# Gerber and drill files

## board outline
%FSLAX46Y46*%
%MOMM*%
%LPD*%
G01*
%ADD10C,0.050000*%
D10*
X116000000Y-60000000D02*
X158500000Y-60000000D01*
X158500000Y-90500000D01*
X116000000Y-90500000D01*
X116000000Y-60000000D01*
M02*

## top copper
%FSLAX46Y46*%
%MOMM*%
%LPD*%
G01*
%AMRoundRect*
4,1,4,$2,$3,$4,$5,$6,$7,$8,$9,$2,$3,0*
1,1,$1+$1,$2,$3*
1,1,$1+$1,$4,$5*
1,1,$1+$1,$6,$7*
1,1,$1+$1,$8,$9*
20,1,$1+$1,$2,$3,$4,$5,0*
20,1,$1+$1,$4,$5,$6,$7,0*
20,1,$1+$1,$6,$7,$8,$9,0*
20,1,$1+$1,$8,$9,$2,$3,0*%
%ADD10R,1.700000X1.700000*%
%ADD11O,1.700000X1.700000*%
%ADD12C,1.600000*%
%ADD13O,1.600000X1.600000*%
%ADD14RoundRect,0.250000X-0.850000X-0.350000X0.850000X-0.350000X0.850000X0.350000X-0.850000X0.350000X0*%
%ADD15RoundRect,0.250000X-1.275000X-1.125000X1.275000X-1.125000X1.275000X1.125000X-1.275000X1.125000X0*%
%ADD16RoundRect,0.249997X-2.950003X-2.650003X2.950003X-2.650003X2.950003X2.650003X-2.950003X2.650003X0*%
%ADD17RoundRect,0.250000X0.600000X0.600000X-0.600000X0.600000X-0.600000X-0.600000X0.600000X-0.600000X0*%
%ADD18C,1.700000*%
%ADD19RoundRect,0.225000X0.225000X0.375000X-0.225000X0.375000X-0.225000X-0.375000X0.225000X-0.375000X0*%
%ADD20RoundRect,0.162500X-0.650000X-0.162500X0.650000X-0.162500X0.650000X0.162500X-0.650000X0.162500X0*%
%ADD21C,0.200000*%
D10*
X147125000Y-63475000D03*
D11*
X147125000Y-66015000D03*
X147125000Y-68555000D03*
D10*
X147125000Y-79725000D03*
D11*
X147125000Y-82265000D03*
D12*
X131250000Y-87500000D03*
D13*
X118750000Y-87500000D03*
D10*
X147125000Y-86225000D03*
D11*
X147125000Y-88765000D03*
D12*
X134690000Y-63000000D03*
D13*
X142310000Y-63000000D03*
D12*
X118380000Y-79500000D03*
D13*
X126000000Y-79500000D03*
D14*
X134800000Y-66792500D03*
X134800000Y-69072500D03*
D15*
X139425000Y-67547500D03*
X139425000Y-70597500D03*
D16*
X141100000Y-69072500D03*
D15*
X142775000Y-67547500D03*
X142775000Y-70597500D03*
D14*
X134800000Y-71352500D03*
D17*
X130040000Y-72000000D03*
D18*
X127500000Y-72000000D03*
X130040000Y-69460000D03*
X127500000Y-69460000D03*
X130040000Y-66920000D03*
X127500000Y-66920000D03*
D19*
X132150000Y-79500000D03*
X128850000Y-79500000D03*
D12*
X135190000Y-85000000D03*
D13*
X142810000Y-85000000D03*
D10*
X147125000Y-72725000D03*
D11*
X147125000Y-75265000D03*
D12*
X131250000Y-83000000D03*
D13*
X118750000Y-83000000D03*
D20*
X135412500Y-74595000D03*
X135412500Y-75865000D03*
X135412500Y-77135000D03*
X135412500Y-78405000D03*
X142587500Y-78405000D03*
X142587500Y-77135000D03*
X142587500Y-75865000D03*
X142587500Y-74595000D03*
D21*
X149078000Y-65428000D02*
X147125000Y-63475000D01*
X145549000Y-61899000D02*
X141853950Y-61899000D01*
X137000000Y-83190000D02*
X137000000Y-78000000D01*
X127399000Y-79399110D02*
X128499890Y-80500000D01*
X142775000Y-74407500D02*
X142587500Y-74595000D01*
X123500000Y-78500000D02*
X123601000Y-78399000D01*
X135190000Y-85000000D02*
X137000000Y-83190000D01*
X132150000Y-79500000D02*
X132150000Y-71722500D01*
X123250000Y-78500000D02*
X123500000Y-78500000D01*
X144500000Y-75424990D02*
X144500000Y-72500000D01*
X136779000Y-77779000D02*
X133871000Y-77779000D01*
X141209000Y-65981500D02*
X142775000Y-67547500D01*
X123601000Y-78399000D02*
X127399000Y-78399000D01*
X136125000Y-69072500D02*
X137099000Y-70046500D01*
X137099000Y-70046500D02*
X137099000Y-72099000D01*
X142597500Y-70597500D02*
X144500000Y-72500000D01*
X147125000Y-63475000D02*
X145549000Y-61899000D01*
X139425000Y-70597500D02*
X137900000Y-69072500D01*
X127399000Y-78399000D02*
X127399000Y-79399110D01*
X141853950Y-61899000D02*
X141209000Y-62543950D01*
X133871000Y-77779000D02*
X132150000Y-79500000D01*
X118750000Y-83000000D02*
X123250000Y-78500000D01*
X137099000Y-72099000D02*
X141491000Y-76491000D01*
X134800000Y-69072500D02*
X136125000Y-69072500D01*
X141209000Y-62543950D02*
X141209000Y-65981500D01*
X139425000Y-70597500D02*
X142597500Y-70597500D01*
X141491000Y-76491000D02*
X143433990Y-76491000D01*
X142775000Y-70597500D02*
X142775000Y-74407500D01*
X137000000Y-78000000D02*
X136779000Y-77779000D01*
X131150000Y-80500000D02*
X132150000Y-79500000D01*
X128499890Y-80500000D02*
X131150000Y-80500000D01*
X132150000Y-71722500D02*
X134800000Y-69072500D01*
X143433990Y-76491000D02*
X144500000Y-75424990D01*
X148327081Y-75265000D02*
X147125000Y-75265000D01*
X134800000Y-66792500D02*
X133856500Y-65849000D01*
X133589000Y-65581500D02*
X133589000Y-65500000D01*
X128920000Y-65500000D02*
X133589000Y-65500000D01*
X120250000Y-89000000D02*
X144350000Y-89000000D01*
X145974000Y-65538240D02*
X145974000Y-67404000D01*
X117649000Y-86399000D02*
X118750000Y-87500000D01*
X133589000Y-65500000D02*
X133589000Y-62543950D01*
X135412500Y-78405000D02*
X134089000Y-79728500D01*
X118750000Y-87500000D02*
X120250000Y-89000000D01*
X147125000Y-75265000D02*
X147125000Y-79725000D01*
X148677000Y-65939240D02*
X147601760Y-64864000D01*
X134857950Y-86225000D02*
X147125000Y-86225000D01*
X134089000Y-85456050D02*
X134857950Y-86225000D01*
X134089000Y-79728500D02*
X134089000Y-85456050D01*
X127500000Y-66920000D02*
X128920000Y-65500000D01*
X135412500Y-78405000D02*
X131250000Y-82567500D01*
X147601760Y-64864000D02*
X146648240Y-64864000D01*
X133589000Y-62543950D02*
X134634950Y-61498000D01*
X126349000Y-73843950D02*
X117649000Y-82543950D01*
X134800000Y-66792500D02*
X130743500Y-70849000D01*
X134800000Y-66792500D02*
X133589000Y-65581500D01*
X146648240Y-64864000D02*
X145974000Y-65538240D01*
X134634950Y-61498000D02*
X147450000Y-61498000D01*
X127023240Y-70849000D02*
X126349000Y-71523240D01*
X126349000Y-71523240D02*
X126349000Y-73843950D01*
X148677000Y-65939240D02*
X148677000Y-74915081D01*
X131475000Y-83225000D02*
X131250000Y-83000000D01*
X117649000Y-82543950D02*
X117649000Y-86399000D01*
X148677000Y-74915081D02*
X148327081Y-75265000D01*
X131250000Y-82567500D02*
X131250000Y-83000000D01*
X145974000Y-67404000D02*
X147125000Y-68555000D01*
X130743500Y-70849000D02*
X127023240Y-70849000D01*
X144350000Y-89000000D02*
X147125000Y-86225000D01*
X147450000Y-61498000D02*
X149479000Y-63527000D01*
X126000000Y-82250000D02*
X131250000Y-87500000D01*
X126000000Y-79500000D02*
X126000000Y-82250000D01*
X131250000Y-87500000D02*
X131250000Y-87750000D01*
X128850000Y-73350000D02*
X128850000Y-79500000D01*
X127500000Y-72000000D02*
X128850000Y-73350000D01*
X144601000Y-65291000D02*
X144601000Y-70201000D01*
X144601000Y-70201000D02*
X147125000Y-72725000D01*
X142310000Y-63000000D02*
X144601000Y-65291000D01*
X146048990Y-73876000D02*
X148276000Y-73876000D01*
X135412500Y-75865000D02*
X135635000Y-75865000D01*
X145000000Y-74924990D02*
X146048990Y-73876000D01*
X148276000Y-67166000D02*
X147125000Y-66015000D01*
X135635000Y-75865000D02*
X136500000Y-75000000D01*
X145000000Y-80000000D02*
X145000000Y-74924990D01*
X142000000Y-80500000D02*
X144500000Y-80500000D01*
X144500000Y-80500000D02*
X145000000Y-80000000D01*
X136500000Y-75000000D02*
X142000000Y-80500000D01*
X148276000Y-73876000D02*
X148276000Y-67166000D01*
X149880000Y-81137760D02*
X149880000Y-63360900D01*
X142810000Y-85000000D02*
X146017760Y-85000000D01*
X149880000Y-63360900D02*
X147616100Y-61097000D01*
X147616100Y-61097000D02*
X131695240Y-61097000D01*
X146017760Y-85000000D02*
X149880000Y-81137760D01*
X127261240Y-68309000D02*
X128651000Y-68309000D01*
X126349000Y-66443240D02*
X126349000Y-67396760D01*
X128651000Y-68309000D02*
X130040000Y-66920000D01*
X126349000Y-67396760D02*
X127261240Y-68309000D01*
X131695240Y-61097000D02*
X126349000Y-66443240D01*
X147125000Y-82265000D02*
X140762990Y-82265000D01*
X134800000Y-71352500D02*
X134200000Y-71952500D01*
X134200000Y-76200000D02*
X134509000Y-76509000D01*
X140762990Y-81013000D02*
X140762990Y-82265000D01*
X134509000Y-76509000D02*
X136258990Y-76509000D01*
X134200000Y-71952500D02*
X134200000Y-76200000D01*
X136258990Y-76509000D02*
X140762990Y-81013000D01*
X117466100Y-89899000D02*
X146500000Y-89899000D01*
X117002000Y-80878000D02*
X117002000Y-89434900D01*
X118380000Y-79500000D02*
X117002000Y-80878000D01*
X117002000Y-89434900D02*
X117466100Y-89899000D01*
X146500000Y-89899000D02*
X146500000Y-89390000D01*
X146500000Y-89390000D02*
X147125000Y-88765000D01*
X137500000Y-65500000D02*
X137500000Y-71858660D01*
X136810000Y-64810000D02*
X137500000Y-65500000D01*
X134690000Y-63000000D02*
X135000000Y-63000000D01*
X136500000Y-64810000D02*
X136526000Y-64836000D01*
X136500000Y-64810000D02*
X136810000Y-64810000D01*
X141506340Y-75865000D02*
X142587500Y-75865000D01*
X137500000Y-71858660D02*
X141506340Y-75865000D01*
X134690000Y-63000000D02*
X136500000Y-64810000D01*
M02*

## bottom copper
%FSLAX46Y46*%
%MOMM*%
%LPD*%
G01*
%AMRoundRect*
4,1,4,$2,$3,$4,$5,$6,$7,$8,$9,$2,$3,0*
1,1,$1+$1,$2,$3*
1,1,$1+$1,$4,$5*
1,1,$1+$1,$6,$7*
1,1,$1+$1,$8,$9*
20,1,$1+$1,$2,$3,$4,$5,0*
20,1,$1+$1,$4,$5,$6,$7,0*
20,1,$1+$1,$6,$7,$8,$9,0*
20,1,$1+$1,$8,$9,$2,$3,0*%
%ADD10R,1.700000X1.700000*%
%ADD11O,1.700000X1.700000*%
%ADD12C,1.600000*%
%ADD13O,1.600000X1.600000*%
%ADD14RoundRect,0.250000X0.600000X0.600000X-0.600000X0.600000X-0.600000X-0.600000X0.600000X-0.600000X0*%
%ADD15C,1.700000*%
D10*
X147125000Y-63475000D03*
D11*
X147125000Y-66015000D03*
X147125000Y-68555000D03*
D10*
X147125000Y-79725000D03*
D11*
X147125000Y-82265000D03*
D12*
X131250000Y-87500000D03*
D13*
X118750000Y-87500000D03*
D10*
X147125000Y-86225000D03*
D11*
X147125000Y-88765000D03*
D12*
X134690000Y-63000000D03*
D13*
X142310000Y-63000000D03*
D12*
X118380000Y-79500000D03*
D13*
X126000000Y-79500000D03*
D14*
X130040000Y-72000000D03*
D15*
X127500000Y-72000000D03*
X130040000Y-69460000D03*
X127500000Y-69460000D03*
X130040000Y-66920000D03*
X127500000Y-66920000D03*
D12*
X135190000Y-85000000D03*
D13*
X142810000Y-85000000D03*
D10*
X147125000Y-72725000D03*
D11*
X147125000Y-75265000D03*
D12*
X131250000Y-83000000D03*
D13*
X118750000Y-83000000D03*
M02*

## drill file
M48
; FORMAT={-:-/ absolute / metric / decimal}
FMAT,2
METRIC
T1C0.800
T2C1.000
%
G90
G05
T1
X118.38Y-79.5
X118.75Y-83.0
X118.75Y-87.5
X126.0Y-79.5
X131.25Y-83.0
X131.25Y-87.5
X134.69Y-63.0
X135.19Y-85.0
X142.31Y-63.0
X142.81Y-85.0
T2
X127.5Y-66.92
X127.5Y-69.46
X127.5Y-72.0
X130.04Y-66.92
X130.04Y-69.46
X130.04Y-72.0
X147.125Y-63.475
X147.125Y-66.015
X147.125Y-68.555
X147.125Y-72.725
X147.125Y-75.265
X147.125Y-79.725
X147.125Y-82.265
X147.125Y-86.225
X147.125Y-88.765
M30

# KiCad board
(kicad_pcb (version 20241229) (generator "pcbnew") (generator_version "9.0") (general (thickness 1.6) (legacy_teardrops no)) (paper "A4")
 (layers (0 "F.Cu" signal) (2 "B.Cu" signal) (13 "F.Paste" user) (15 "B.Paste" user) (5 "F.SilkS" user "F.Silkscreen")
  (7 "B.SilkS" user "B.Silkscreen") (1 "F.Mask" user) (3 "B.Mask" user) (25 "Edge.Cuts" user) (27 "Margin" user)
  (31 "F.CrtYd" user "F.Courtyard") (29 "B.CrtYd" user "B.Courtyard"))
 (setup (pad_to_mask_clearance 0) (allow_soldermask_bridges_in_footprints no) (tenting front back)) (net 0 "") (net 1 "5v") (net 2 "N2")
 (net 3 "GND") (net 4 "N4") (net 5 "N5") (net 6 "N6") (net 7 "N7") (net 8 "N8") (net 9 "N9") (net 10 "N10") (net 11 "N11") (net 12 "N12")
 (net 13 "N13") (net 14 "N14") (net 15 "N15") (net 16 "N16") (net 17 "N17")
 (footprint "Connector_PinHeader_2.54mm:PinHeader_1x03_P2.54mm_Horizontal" (layer "F.Cu") (at 147.125 63.475)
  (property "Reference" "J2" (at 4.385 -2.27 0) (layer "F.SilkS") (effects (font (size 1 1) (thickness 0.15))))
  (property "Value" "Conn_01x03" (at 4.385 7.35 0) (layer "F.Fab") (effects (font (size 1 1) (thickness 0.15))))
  (pad "1" thru_hole rect (at 0 0) (size 1.7 1.7) (drill 1) (layers "*.Cu" "*.Mask") (remove_unused_layers no) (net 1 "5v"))
  (pad "2" thru_hole oval (at 0 2.54) (size 1.7 1.7) (drill 1) (layers "*.Cu" "*.Mask") (remove_unused_layers no) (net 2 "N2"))
  (pad "3" thru_hole oval (at 0 5.08) (size 1.7 1.7) (drill 1) (layers "*.Cu" "*.Mask") (remove_unused_layers no) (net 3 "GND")))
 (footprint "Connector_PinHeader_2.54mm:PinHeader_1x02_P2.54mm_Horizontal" (layer "F.Cu") (at 147.125 79.725)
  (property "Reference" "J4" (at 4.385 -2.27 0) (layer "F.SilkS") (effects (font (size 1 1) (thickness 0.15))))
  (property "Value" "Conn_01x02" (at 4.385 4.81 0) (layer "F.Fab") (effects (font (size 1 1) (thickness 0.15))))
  (pad "1" thru_hole rect (at 0 0) (size 1.7 1.7) (drill 1) (layers "*.Cu" "*.Mask") (remove_unused_layers no) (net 3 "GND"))
  (pad "2" thru_hole oval (at 0 2.54) (size 1.7 1.7) (drill 1) (layers "*.Cu" "*.Mask") (remove_unused_layers no) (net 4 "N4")))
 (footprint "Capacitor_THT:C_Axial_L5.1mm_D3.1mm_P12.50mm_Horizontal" (layer "F.Cu") (at 131.25 87.5 180)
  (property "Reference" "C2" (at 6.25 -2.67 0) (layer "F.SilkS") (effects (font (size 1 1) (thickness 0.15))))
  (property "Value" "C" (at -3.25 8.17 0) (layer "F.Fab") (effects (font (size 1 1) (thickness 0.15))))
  (pad "1" thru_hole circle (at 0 0 180) (size 1.6 1.6) (drill 0.8) (layers "*.Cu" "*.Mask") (remove_unused_layers no) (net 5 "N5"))
  (pad "2" thru_hole oval (at 12.5 0 180) (size 1.6 1.6) (drill 0.8) (layers "*.Cu" "*.Mask") (remove_unused_layers no) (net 3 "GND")))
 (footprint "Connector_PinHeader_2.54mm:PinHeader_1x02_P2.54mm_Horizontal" (layer "F.Cu") (at 147.125 86.225)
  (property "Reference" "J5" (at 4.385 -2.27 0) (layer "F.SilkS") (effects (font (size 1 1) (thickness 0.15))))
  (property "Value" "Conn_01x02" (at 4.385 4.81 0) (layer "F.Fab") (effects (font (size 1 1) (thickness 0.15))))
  (pad "1" thru_hole rect (at 0 0) (size 1.7 1.7) (drill 1) (layers "*.Cu" "*.Mask") (remove_unused_layers no) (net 3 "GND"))
  (pad "2" thru_hole oval (at 0 2.54) (size 1.7 1.7) (drill 1) (layers "*.Cu" "*.Mask") (remove_unused_layers no) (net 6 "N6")))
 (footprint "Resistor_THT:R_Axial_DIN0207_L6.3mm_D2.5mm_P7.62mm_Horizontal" (layer "F.Cu") (at 134.69 63)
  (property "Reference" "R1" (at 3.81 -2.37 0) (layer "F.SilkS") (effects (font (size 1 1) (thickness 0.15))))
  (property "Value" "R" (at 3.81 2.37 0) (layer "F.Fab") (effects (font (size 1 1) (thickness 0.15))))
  (pad "1" thru_hole circle (at 0 0) (size 1.6 1.6) (drill 0.8) (layers "*.Cu" "*.Mask") (remove_unused_layers no) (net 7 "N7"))
  (pad "2" thru_hole oval (at 7.62 0) (size 1.6 1.6) (drill 0.8) (layers "*.Cu" "*.Mask") (remove_unused_layers no) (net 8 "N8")))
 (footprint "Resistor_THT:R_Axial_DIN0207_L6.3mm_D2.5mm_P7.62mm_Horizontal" (layer "F.Cu") (at 118.38 79.5)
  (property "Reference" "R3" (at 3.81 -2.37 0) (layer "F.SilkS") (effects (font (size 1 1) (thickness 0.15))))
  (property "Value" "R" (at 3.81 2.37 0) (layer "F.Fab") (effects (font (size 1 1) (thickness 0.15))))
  (pad "1" thru_hole circle (at 0 0) (size 1.6 1.6) (drill 0.8) (layers "*.Cu" "*.Mask") (remove_unused_layers no) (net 6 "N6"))
  (pad "2" thru_hole oval (at 7.62 0) (size 1.6 1.6) (drill 0.8) (layers "*.Cu" "*.Mask") (remove_unused_layers no) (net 5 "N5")))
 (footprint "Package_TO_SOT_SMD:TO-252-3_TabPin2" (layer "F.Cu") (at 139.84 69.0725)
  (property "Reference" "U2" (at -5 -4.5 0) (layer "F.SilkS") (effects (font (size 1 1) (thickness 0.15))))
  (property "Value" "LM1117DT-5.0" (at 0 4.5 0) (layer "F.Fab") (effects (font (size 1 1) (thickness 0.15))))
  (pad "1" smd roundrect (at -5.04 -2.28) (size 2.2 1.2) (layers "F.Cu" "F.Mask" "F.Paste") (roundrect_rratio 0.208333) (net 3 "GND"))
  (pad "2" smd roundrect (at -5.04 0) (size 2.2 1.2) (layers "F.Cu" "F.Mask" "F.Paste") (roundrect_rratio 0.208333) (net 1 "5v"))
  (pad "2" smd roundrect (at -0.415 -1.525) (size 3.05 2.75) (layers "F.Cu" "F.Paste") (roundrect_rratio 0.090909) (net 1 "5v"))
  (pad "2" smd roundrect (at -0.415 1.525) (size 3.05 2.75) (layers "F.Cu" "F.Paste") (roundrect_rratio 0.090909) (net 1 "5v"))
  (pad "2" smd roundrect (at 1.26 0) (size 6.4 5.8) (layers "F.Cu" "F.Mask") (roundrect_rratio 0.043103) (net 1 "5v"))
  (pad "2" smd roundrect (at 2.935 -1.525) (size 3.05 2.75) (layers "F.Cu" "F.Paste") (roundrect_rratio 0.090909) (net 1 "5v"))
  (pad "2" smd roundrect (at 2.935 1.525) (size 3.05 2.75) (layers "F.Cu" "F.Paste") (roundrect_rratio 0.090909) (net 1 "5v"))
  (pad "3" smd roundrect (at -5.04 2.28) (size 2.2 1.2) (layers "F.Cu" "F.Mask" "F.Paste") (roundrect_rratio 0.208333) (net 4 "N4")))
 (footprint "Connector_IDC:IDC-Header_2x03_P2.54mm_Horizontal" (layer "F.Cu") (at 130.04 72 180)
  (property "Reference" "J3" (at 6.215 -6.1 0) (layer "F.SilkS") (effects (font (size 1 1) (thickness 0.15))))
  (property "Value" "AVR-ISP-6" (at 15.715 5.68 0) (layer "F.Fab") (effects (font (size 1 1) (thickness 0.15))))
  (pad "1" thru_hole roundrect (at 0 0 180) (size 1.7 1.7) (drill 1) (layers "*.Cu" "*.Mask") (remove_unused_layers no)
   (roundrect_rratio 0.147059) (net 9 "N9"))
  (pad "2" thru_hole circle (at 2.54 0 180) (size 1.7 1.7) (drill 1) (layers "*.Cu" "*.Mask") (remove_unused_layers no) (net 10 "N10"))
  (pad "3" thru_hole circle (at 0 2.54 180) (size 1.7 1.7) (drill 1) (layers "*.Cu" "*.Mask") (remove_unused_layers no) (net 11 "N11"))
  (pad "4" thru_hole circle (at 2.54 2.54 180) (size 1.7 1.7) (drill 1) (layers "*.Cu" "*.Mask") (remove_unused_layers no) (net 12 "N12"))
  (pad "5" thru_hole circle (at 0 5.08 180) (size 1.7 1.7) (drill 1) (layers "*.Cu" "*.Mask") (remove_unused_layers no) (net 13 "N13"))
  (pad "6" thru_hole circle (at 2.54 5.08 180) (size 1.7 1.7) (drill 1) (layers "*.Cu" "*.Mask") (remove_unused_layers no) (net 3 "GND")))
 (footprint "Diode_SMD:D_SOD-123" (layer "F.Cu") (at 130.5 79.5 180)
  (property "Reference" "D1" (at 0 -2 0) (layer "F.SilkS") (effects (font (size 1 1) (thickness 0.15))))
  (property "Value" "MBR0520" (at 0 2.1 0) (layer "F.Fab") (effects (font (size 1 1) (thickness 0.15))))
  (pad "1" smd roundrect (at -1.65 0 180) (size 0.9 1.2) (layers "F.Cu" "F.Mask" "F.Paste") (roundrect_rratio 0.25) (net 1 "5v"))
  (pad "2" smd roundrect (at 1.65 0 180) (size 0.9 1.2) (layers "F.Cu" "F.Mask" "F.Paste") (roundrect_rratio 0.25) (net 10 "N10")))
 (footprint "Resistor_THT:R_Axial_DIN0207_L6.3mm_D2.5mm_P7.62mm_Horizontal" (layer "F.Cu") (at 135.19 85)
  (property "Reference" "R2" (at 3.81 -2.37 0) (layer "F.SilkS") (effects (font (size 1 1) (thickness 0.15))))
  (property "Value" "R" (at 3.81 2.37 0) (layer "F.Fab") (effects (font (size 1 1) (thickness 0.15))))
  (pad "1" thru_hole circle (at 0 0) (size 1.6 1.6) (drill 0.8) (layers "*.Cu" "*.Mask") (remove_unused_layers no) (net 1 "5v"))
  (pad "2" thru_hole oval (at 7.62 0) (size 1.6 1.6) (drill 0.8) (layers "*.Cu" "*.Mask") (remove_unused_layers no) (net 13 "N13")))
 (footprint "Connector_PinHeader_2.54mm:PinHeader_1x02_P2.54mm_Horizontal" (layer "F.Cu") (at 147.125 72.725)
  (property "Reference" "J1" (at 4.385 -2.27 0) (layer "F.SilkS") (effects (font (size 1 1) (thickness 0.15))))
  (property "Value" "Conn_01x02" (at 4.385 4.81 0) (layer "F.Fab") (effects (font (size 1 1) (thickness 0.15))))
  (pad "1" thru_hole rect (at 0 0) (size 1.7 1.7) (drill 1) (layers "*.Cu" "*.Mask") (remove_unused_layers no) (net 8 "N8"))
  (pad "2" thru_hole oval (at 0 2.54) (size 1.7 1.7) (drill 1) (layers "*.Cu" "*.Mask") (remove_unused_layers no) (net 3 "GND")))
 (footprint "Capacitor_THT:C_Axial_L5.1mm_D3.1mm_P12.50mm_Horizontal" (layer "F.Cu") (at 131.25 83 180)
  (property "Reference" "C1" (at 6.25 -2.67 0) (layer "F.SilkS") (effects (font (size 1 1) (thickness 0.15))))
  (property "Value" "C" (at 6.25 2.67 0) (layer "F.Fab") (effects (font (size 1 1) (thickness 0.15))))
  (pad "1" thru_hole circle (at 0 0 180) (size 1.6 1.6) (drill 0.8) (layers "*.Cu" "*.Mask") (remove_unused_layers no) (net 3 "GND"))
  (pad "2" thru_hole oval (at 12.5 0 180) (size 1.6 1.6) (drill 0.8) (layers "*.Cu" "*.Mask") (remove_unused_layers no) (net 1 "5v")))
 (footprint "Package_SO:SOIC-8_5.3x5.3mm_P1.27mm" (layer "F.Cu") (at 139 76.5)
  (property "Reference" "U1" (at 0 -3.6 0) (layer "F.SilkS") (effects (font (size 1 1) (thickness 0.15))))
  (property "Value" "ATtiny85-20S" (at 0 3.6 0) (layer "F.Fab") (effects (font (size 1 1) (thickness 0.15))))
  (pad "1" smd roundrect (at -3.5875 -1.905) (size 1.625 0.65) (layers "F.Cu" "F.Mask" "F.Paste") (roundrect_rratio 0.25) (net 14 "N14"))
  (pad "2" smd roundrect (at -3.5875 -0.635) (size 1.625 0.65) (layers "F.Cu" "F.Mask" "F.Paste") (roundrect_rratio 0.25) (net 2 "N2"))
  (pad "3" smd roundrect (at -3.5875 0.635) (size 1.625 0.65) (layers "F.Cu" "F.Mask" "F.Paste") (roundrect_rratio 0.25) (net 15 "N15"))
  (pad "4" smd roundrect (at -3.5875 1.905) (size 1.625 0.65) (layers "F.Cu" "F.Mask" "F.Paste") (roundrect_rratio 0.25) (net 3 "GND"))
  (pad "5" smd roundrect (at 3.5875 1.905) (size 1.625 0.65) (layers "F.Cu" "F.Mask" "F.Paste") (roundrect_rratio 0.25) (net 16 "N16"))
  (pad "6" smd roundrect (at 3.5875 0.635) (size 1.625 0.65) (layers "F.Cu" "F.Mask" "F.Paste") (roundrect_rratio 0.25) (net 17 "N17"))
  (pad "7" smd roundrect (at 3.5875 -0.635) (size 1.625 0.65) (layers "F.Cu" "F.Mask" "F.Paste") (roundrect_rratio 0.25) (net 7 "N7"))
  (pad "8" smd roundrect (at 3.5875 -1.905) (size 1.625 0.65) (layers "F.Cu" "F.Mask" "F.Paste") (roundrect_rratio 0.25) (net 1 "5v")))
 (gr_rect (start 116 60) (end 158.5 90.5) (stroke (width 0.05) (type default)) (fill no) (layer "Edge.Cuts"))
 (segment (start 149.078 65.428) (end 147.125 63.475) (width 0.2) (layer "F.Cu") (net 1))
 (segment (start 145.549 61.899) (end 141.85395 61.899) (width 0.2) (layer "F.Cu") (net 1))
 (segment (start 137 83.19) (end 137 78) (width 0.2) (layer "F.Cu") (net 1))
 (segment (start 127.399 79.39911) (end 128.49989 80.5) (width 0.2) (layer "F.Cu") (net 1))
 (segment (start 142.775 74.4075) (end 142.5875 74.595) (width 0.2) (layer "F.Cu") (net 1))
 (segment (start 123.5 78.5) (end 123.601 78.399) (width 0.2) (layer "F.Cu") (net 1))
 (segment (start 135.19 85) (end 137 83.19) (width 0.2) (layer "F.Cu") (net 1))
 (segment (start 132.15 79.5) (end 132.15 71.7225) (width 0.2) (layer "F.Cu") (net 1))
 (segment (start 123.25 78.5) (end 123.5 78.5) (width 0.2) (layer "F.Cu") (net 1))
 (segment (start 144.5 75.42499) (end 144.5 72.5) (width 0.2) (layer "F.Cu") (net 1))
 (segment (start 136.779 77.779) (end 133.871 77.779) (width 0.2) (layer "F.Cu") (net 1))
 (segment (start 141.209 65.9815) (end 142.775 67.5475) (width 0.2) (layer "F.Cu") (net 1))
 (segment (start 123.601 78.399) (end 127.399 78.399) (width 0.2) (layer "F.Cu") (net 1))
 (segment (start 136.125 69.0725) (end 137.099 70.0465) (width 0.2) (layer "F.Cu") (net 1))
 (segment (start 137.099 70.0465) (end 137.099 72.099) (width 0.2) (layer "F.Cu") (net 1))
 (segment (start 142.5975 70.5975) (end 144.5 72.5) (width 0.2) (layer "F.Cu") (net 1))
 (segment (start 147.125 63.475) (end 145.549 61.899) (width 0.2) (layer "F.Cu") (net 1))
 (segment (start 139.425 70.5975) (end 137.9 69.0725) (width 0.2) (layer "F.Cu") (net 1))
 (segment (start 127.399 78.399) (end 127.399 79.39911) (width 0.2) (layer "F.Cu") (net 1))
 (segment (start 141.85395 61.899) (end 141.209 62.54395) (width 0.2) (layer "F.Cu") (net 1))
 (segment (start 133.871 77.779) (end 132.15 79.5) (width 0.2) (layer "F.Cu") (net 1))
 (segment (start 118.75 83) (end 123.25 78.5) (width 0.2) (layer "F.Cu") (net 1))
 (segment (start 137.099 72.099) (end 141.491 76.491) (width 0.2) (layer "F.Cu") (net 1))
 (segment (start 134.8 69.0725) (end 136.125 69.0725) (width 0.2) (layer "F.Cu") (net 1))
 (segment (start 141.209 62.54395) (end 141.209 65.9815) (width 0.2) (layer "F.Cu") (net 1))
 (segment (start 139.425 70.5975) (end 142.5975 70.5975) (width 0.2) (layer "F.Cu") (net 1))
 (segment (start 141.491 76.491) (end 143.43399 76.491) (width 0.2) (layer "F.Cu") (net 1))
 (segment (start 142.775 70.5975) (end 142.775 74.4075) (width 0.2) (layer "F.Cu") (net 1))
 (segment (start 137 78) (end 136.779 77.779) (width 0.2) (layer "F.Cu") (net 1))
 (segment (start 131.15 80.5) (end 132.15 79.5) (width 0.2) (layer "F.Cu") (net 1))
 (segment (start 128.49989 80.5) (end 131.15 80.5) (width 0.2) (layer "F.Cu") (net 1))
 (segment (start 132.15 71.7225) (end 134.8 69.0725) (width 0.2) (layer "F.Cu") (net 1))
 (segment (start 143.43399 76.491) (end 144.5 75.42499) (width 0.2) (layer "F.Cu") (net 1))
 (segment (start 148.327081 75.265) (end 147.125 75.265) (width 0.2) (layer "F.Cu") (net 3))
 (segment (start 134.8 66.7925) (end 133.8565 65.849) (width 0.2) (layer "F.Cu") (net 3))
 (segment (start 133.589 65.5815) (end 133.589 65.5) (width 0.2) (layer "F.Cu") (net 3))
 (segment (start 128.92 65.5) (end 133.589 65.5) (width 0.2) (layer "F.Cu") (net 3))
 (segment (start 120.25 89) (end 144.35 89) (width 0.2) (layer "F.Cu") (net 3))
 (segment (start 145.974 65.53824) (end 145.974 67.404) (width 0.2) (layer "F.Cu") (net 3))
 (segment (start 117.649 86.399) (end 118.75 87.5) (width 0.2) (layer "F.Cu") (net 3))
 (segment (start 133.589 65.5) (end 133.589 62.54395) (width 0.2) (layer "F.Cu") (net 3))
 (segment (start 135.4125 78.405) (end 134.089 79.7285) (width 0.2) (layer "F.Cu") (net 3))
 (segment (start 118.75 87.5) (end 120.25 89) (width 0.2) (layer "F.Cu") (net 3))
 (segment (start 147.125 75.265) (end 147.125 79.725) (width 0.2) (layer "F.Cu") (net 3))
 (segment (start 148.677 65.93924) (end 147.60176 64.864) (width 0.2) (layer "F.Cu") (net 3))
 (segment (start 134.85795 86.225) (end 147.125 86.225) (width 0.2) (layer "F.Cu") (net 3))
 (segment (start 134.089 85.45605) (end 134.85795 86.225) (width 0.2) (layer "F.Cu") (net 3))
 (segment (start 134.089 79.7285) (end 134.089 85.45605) (width 0.2) (layer "F.Cu") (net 3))
 (segment (start 127.5 66.92) (end 128.92 65.5) (width 0.2) (layer "F.Cu") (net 3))
 (segment (start 135.4125 78.405) (end 131.25 82.5675) (width 0.2) (layer "F.Cu") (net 3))
 (segment (start 147.60176 64.864) (end 146.64824 64.864) (width 0.2) (layer "F.Cu") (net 3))
 (segment (start 133.589 62.54395) (end 134.63495 61.498) (width 0.2) (layer "F.Cu") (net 3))
 (segment (start 126.349 73.84395) (end 117.649 82.54395) (width 0.2) (layer "F.Cu") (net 3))
 (segment (start 134.8 66.7925) (end 130.7435 70.849) (width 0.2) (layer "F.Cu") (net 3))
 (segment (start 134.8 66.7925) (end 133.589 65.5815) (width 0.2) (layer "F.Cu") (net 3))
 (segment (start 146.64824 64.864) (end 145.974 65.53824) (width 0.2) (layer "F.Cu") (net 3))
 (segment (start 134.63495 61.498) (end 147.45 61.498) (width 0.2) (layer "F.Cu") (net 3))
 (segment (start 127.02324 70.849) (end 126.349 71.52324) (width 0.2) (layer "F.Cu") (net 3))
 (segment (start 126.349 71.52324) (end 126.349 73.84395) (width 0.2) (layer "F.Cu") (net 3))
 (segment (start 148.677 65.93924) (end 148.677 74.915081) (width 0.2) (layer "F.Cu") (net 3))
 (segment (start 131.475 83.225) (end 131.25 83) (width 0.2) (layer "F.Cu") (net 3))
 (segment (start 117.649 82.54395) (end 117.649 86.399) (width 0.2) (layer "F.Cu") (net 3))
 (segment (start 148.677 74.915081) (end 148.327081 75.265) (width 0.2) (layer "F.Cu") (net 3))
 (segment (start 131.25 82.5675) (end 131.25 83) (width 0.2) (layer "F.Cu") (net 3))
 (segment (start 145.974 67.404) (end 147.125 68.555) (width 0.2) (layer "F.Cu") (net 3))
 (segment (start 130.7435 70.849) (end 127.02324 70.849) (width 0.2) (layer "F.Cu") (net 3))
 (segment (start 144.35 89) (end 147.125 86.225) (width 0.2) (layer "F.Cu") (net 3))
 (segment (start 147.45 61.498) (end 149.479 63.527) (width 0.2) (layer "F.Cu") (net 3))
 (segment (start 126 82.25) (end 131.25 87.5) (width 0.2) (layer "F.Cu") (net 5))
 (segment (start 126 79.5) (end 126 82.25) (width 0.2) (layer "F.Cu") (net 5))
 (segment (start 131.25 87.5) (end 131.25 87.75) (width 0.2) (layer "F.Cu") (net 5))
 (segment (start 128.85 73.35) (end 128.85 79.5) (width 0.2) (layer "F.Cu") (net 10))
 (segment (start 127.5 72) (end 128.85 73.35) (width 0.2) (layer "F.Cu") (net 10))
 (segment (start 144.601 65.291) (end 144.601 70.201) (width 0.2) (layer "F.Cu") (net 8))
 (segment (start 144.601 70.201) (end 147.125 72.725) (width 0.2) (layer "F.Cu") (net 8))
 (segment (start 142.31 63) (end 144.601 65.291) (width 0.2) (layer "F.Cu") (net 8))
 (segment (start 146.04899 73.876) (end 148.276 73.876) (width 0.2) (layer "F.Cu") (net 2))
 (segment (start 135.4125 75.865) (end 135.635 75.865) (width 0.2) (layer "F.Cu") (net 2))
 (segment (start 145 74.92499) (end 146.04899 73.876) (width 0.2) (layer "F.Cu") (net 2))
 (segment (start 148.276 67.166) (end 147.125 66.015) (width 0.2) (layer "F.Cu") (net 2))
 (segment (start 135.635 75.865) (end 136.5 75) (width 0.2) (layer "F.Cu") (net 2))
 (segment (start 145 80) (end 145 74.92499) (width 0.2) (layer "F.Cu") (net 2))
 (segment (start 142 80.5) (end 144.5 80.5) (width 0.2) (layer "F.Cu") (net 2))
 (segment (start 144.5 80.5) (end 145 80) (width 0.2) (layer "F.Cu") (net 2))
 (segment (start 136.5 75) (end 142 80.5) (width 0.2) (layer "F.Cu") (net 2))
 (segment (start 148.276 73.876) (end 148.276 67.166) (width 0.2) (layer "F.Cu") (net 2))
 (segment (start 149.88 81.13776) (end 149.88 63.3609) (width 0.2) (layer "F.Cu") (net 13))
 (segment (start 142.81 85) (end 146.01776 85) (width 0.2) (layer "F.Cu") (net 13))
 (segment (start 149.88 63.3609) (end 147.6161 61.097) (width 0.2) (layer "F.Cu") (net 13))
 (segment (start 147.6161 61.097) (end 131.69524 61.097) (width 0.2) (layer "F.Cu") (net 13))
 (segment (start 146.01776 85) (end 149.88 81.13776) (width 0.2) (layer "F.Cu") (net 13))
 (segment (start 127.26124 68.309) (end 128.651 68.309) (width 0.2) (layer "F.Cu") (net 13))
 (segment (start 126.349 66.44324) (end 126.349 67.39676) (width 0.2) (layer "F.Cu") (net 13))
 (segment (start 128.651 68.309) (end 130.04 66.92) (width 0.2) (layer "F.Cu") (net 13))
 (segment (start 126.349 67.39676) (end 127.26124 68.309) (width 0.2) (layer "F.Cu") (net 13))
 (segment (start 131.69524 61.097) (end 126.349 66.44324) (width 0.2) (layer "F.Cu") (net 13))
 (segment (start 147.125 82.265) (end 140.76299 82.265) (width 0.2) (layer "F.Cu") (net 4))
 (segment (start 134.8 71.3525) (end 134.2 71.9525) (width 0.2) (layer "F.Cu") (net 4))
 (segment (start 134.2 76.2) (end 134.509 76.509) (width 0.2) (layer "F.Cu") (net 4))
 (segment (start 140.76299 81.013) (end 140.76299 82.265) (width 0.2) (layer "F.Cu") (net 4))
 (segment (start 134.509 76.509) (end 136.25899 76.509) (width 0.2) (layer "F.Cu") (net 4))
 (segment (start 134.2 71.9525) (end 134.2 76.2) (width 0.2) (layer "F.Cu") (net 4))
 (segment (start 136.25899 76.509) (end 140.76299 81.013) (width 0.2) (layer "F.Cu") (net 4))
 (segment (start 117.4661 89.899) (end 146.5 89.899) (width 0.2) (layer "F.Cu") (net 6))
 (segment (start 117.002 80.878) (end 117.002 89.4349) (width 0.2) (layer "F.Cu") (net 6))
 (segment (start 118.38 79.5) (end 117.002 80.878) (width 0.2) (layer "F.Cu") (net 6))
 (segment (start 117.002 89.4349) (end 117.4661 89.899) (width 0.2) (layer "F.Cu") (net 6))
 (segment (start 146.5 89.899) (end 146.5 89.39) (width 0.2) (layer "F.Cu") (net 6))
 (segment (start 146.5 89.39) (end 147.125 88.765) (width 0.2) (layer "F.Cu") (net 6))
 (segment (start 137.5 65.5) (end 137.5 71.85866) (width 0.2) (layer "F.Cu") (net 7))
 (segment (start 136.81 64.81) (end 137.5 65.5) (width 0.2) (layer "F.Cu") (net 7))
 (segment (start 134.69 63) (end 135 63) (width 0.2) (layer "F.Cu") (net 7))
 (segment (start 136.5 64.81) (end 136.526 64.836) (width 0.2) (layer "F.Cu") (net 7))
 (segment (start 136.5 64.81) (end 136.81 64.81) (width 0.2) (layer "F.Cu") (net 7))
 (segment (start 141.50634 75.865) (end 142.5875 75.865) (width 0.2) (layer "F.Cu") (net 7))
 (segment (start 137.5 71.85866) (end 141.50634 75.865) (width 0.2) (layer "F.Cu") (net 7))
 (segment (start 134.69 63) (end 136.5 64.81) (width 0.2) (layer "F.Cu") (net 7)))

